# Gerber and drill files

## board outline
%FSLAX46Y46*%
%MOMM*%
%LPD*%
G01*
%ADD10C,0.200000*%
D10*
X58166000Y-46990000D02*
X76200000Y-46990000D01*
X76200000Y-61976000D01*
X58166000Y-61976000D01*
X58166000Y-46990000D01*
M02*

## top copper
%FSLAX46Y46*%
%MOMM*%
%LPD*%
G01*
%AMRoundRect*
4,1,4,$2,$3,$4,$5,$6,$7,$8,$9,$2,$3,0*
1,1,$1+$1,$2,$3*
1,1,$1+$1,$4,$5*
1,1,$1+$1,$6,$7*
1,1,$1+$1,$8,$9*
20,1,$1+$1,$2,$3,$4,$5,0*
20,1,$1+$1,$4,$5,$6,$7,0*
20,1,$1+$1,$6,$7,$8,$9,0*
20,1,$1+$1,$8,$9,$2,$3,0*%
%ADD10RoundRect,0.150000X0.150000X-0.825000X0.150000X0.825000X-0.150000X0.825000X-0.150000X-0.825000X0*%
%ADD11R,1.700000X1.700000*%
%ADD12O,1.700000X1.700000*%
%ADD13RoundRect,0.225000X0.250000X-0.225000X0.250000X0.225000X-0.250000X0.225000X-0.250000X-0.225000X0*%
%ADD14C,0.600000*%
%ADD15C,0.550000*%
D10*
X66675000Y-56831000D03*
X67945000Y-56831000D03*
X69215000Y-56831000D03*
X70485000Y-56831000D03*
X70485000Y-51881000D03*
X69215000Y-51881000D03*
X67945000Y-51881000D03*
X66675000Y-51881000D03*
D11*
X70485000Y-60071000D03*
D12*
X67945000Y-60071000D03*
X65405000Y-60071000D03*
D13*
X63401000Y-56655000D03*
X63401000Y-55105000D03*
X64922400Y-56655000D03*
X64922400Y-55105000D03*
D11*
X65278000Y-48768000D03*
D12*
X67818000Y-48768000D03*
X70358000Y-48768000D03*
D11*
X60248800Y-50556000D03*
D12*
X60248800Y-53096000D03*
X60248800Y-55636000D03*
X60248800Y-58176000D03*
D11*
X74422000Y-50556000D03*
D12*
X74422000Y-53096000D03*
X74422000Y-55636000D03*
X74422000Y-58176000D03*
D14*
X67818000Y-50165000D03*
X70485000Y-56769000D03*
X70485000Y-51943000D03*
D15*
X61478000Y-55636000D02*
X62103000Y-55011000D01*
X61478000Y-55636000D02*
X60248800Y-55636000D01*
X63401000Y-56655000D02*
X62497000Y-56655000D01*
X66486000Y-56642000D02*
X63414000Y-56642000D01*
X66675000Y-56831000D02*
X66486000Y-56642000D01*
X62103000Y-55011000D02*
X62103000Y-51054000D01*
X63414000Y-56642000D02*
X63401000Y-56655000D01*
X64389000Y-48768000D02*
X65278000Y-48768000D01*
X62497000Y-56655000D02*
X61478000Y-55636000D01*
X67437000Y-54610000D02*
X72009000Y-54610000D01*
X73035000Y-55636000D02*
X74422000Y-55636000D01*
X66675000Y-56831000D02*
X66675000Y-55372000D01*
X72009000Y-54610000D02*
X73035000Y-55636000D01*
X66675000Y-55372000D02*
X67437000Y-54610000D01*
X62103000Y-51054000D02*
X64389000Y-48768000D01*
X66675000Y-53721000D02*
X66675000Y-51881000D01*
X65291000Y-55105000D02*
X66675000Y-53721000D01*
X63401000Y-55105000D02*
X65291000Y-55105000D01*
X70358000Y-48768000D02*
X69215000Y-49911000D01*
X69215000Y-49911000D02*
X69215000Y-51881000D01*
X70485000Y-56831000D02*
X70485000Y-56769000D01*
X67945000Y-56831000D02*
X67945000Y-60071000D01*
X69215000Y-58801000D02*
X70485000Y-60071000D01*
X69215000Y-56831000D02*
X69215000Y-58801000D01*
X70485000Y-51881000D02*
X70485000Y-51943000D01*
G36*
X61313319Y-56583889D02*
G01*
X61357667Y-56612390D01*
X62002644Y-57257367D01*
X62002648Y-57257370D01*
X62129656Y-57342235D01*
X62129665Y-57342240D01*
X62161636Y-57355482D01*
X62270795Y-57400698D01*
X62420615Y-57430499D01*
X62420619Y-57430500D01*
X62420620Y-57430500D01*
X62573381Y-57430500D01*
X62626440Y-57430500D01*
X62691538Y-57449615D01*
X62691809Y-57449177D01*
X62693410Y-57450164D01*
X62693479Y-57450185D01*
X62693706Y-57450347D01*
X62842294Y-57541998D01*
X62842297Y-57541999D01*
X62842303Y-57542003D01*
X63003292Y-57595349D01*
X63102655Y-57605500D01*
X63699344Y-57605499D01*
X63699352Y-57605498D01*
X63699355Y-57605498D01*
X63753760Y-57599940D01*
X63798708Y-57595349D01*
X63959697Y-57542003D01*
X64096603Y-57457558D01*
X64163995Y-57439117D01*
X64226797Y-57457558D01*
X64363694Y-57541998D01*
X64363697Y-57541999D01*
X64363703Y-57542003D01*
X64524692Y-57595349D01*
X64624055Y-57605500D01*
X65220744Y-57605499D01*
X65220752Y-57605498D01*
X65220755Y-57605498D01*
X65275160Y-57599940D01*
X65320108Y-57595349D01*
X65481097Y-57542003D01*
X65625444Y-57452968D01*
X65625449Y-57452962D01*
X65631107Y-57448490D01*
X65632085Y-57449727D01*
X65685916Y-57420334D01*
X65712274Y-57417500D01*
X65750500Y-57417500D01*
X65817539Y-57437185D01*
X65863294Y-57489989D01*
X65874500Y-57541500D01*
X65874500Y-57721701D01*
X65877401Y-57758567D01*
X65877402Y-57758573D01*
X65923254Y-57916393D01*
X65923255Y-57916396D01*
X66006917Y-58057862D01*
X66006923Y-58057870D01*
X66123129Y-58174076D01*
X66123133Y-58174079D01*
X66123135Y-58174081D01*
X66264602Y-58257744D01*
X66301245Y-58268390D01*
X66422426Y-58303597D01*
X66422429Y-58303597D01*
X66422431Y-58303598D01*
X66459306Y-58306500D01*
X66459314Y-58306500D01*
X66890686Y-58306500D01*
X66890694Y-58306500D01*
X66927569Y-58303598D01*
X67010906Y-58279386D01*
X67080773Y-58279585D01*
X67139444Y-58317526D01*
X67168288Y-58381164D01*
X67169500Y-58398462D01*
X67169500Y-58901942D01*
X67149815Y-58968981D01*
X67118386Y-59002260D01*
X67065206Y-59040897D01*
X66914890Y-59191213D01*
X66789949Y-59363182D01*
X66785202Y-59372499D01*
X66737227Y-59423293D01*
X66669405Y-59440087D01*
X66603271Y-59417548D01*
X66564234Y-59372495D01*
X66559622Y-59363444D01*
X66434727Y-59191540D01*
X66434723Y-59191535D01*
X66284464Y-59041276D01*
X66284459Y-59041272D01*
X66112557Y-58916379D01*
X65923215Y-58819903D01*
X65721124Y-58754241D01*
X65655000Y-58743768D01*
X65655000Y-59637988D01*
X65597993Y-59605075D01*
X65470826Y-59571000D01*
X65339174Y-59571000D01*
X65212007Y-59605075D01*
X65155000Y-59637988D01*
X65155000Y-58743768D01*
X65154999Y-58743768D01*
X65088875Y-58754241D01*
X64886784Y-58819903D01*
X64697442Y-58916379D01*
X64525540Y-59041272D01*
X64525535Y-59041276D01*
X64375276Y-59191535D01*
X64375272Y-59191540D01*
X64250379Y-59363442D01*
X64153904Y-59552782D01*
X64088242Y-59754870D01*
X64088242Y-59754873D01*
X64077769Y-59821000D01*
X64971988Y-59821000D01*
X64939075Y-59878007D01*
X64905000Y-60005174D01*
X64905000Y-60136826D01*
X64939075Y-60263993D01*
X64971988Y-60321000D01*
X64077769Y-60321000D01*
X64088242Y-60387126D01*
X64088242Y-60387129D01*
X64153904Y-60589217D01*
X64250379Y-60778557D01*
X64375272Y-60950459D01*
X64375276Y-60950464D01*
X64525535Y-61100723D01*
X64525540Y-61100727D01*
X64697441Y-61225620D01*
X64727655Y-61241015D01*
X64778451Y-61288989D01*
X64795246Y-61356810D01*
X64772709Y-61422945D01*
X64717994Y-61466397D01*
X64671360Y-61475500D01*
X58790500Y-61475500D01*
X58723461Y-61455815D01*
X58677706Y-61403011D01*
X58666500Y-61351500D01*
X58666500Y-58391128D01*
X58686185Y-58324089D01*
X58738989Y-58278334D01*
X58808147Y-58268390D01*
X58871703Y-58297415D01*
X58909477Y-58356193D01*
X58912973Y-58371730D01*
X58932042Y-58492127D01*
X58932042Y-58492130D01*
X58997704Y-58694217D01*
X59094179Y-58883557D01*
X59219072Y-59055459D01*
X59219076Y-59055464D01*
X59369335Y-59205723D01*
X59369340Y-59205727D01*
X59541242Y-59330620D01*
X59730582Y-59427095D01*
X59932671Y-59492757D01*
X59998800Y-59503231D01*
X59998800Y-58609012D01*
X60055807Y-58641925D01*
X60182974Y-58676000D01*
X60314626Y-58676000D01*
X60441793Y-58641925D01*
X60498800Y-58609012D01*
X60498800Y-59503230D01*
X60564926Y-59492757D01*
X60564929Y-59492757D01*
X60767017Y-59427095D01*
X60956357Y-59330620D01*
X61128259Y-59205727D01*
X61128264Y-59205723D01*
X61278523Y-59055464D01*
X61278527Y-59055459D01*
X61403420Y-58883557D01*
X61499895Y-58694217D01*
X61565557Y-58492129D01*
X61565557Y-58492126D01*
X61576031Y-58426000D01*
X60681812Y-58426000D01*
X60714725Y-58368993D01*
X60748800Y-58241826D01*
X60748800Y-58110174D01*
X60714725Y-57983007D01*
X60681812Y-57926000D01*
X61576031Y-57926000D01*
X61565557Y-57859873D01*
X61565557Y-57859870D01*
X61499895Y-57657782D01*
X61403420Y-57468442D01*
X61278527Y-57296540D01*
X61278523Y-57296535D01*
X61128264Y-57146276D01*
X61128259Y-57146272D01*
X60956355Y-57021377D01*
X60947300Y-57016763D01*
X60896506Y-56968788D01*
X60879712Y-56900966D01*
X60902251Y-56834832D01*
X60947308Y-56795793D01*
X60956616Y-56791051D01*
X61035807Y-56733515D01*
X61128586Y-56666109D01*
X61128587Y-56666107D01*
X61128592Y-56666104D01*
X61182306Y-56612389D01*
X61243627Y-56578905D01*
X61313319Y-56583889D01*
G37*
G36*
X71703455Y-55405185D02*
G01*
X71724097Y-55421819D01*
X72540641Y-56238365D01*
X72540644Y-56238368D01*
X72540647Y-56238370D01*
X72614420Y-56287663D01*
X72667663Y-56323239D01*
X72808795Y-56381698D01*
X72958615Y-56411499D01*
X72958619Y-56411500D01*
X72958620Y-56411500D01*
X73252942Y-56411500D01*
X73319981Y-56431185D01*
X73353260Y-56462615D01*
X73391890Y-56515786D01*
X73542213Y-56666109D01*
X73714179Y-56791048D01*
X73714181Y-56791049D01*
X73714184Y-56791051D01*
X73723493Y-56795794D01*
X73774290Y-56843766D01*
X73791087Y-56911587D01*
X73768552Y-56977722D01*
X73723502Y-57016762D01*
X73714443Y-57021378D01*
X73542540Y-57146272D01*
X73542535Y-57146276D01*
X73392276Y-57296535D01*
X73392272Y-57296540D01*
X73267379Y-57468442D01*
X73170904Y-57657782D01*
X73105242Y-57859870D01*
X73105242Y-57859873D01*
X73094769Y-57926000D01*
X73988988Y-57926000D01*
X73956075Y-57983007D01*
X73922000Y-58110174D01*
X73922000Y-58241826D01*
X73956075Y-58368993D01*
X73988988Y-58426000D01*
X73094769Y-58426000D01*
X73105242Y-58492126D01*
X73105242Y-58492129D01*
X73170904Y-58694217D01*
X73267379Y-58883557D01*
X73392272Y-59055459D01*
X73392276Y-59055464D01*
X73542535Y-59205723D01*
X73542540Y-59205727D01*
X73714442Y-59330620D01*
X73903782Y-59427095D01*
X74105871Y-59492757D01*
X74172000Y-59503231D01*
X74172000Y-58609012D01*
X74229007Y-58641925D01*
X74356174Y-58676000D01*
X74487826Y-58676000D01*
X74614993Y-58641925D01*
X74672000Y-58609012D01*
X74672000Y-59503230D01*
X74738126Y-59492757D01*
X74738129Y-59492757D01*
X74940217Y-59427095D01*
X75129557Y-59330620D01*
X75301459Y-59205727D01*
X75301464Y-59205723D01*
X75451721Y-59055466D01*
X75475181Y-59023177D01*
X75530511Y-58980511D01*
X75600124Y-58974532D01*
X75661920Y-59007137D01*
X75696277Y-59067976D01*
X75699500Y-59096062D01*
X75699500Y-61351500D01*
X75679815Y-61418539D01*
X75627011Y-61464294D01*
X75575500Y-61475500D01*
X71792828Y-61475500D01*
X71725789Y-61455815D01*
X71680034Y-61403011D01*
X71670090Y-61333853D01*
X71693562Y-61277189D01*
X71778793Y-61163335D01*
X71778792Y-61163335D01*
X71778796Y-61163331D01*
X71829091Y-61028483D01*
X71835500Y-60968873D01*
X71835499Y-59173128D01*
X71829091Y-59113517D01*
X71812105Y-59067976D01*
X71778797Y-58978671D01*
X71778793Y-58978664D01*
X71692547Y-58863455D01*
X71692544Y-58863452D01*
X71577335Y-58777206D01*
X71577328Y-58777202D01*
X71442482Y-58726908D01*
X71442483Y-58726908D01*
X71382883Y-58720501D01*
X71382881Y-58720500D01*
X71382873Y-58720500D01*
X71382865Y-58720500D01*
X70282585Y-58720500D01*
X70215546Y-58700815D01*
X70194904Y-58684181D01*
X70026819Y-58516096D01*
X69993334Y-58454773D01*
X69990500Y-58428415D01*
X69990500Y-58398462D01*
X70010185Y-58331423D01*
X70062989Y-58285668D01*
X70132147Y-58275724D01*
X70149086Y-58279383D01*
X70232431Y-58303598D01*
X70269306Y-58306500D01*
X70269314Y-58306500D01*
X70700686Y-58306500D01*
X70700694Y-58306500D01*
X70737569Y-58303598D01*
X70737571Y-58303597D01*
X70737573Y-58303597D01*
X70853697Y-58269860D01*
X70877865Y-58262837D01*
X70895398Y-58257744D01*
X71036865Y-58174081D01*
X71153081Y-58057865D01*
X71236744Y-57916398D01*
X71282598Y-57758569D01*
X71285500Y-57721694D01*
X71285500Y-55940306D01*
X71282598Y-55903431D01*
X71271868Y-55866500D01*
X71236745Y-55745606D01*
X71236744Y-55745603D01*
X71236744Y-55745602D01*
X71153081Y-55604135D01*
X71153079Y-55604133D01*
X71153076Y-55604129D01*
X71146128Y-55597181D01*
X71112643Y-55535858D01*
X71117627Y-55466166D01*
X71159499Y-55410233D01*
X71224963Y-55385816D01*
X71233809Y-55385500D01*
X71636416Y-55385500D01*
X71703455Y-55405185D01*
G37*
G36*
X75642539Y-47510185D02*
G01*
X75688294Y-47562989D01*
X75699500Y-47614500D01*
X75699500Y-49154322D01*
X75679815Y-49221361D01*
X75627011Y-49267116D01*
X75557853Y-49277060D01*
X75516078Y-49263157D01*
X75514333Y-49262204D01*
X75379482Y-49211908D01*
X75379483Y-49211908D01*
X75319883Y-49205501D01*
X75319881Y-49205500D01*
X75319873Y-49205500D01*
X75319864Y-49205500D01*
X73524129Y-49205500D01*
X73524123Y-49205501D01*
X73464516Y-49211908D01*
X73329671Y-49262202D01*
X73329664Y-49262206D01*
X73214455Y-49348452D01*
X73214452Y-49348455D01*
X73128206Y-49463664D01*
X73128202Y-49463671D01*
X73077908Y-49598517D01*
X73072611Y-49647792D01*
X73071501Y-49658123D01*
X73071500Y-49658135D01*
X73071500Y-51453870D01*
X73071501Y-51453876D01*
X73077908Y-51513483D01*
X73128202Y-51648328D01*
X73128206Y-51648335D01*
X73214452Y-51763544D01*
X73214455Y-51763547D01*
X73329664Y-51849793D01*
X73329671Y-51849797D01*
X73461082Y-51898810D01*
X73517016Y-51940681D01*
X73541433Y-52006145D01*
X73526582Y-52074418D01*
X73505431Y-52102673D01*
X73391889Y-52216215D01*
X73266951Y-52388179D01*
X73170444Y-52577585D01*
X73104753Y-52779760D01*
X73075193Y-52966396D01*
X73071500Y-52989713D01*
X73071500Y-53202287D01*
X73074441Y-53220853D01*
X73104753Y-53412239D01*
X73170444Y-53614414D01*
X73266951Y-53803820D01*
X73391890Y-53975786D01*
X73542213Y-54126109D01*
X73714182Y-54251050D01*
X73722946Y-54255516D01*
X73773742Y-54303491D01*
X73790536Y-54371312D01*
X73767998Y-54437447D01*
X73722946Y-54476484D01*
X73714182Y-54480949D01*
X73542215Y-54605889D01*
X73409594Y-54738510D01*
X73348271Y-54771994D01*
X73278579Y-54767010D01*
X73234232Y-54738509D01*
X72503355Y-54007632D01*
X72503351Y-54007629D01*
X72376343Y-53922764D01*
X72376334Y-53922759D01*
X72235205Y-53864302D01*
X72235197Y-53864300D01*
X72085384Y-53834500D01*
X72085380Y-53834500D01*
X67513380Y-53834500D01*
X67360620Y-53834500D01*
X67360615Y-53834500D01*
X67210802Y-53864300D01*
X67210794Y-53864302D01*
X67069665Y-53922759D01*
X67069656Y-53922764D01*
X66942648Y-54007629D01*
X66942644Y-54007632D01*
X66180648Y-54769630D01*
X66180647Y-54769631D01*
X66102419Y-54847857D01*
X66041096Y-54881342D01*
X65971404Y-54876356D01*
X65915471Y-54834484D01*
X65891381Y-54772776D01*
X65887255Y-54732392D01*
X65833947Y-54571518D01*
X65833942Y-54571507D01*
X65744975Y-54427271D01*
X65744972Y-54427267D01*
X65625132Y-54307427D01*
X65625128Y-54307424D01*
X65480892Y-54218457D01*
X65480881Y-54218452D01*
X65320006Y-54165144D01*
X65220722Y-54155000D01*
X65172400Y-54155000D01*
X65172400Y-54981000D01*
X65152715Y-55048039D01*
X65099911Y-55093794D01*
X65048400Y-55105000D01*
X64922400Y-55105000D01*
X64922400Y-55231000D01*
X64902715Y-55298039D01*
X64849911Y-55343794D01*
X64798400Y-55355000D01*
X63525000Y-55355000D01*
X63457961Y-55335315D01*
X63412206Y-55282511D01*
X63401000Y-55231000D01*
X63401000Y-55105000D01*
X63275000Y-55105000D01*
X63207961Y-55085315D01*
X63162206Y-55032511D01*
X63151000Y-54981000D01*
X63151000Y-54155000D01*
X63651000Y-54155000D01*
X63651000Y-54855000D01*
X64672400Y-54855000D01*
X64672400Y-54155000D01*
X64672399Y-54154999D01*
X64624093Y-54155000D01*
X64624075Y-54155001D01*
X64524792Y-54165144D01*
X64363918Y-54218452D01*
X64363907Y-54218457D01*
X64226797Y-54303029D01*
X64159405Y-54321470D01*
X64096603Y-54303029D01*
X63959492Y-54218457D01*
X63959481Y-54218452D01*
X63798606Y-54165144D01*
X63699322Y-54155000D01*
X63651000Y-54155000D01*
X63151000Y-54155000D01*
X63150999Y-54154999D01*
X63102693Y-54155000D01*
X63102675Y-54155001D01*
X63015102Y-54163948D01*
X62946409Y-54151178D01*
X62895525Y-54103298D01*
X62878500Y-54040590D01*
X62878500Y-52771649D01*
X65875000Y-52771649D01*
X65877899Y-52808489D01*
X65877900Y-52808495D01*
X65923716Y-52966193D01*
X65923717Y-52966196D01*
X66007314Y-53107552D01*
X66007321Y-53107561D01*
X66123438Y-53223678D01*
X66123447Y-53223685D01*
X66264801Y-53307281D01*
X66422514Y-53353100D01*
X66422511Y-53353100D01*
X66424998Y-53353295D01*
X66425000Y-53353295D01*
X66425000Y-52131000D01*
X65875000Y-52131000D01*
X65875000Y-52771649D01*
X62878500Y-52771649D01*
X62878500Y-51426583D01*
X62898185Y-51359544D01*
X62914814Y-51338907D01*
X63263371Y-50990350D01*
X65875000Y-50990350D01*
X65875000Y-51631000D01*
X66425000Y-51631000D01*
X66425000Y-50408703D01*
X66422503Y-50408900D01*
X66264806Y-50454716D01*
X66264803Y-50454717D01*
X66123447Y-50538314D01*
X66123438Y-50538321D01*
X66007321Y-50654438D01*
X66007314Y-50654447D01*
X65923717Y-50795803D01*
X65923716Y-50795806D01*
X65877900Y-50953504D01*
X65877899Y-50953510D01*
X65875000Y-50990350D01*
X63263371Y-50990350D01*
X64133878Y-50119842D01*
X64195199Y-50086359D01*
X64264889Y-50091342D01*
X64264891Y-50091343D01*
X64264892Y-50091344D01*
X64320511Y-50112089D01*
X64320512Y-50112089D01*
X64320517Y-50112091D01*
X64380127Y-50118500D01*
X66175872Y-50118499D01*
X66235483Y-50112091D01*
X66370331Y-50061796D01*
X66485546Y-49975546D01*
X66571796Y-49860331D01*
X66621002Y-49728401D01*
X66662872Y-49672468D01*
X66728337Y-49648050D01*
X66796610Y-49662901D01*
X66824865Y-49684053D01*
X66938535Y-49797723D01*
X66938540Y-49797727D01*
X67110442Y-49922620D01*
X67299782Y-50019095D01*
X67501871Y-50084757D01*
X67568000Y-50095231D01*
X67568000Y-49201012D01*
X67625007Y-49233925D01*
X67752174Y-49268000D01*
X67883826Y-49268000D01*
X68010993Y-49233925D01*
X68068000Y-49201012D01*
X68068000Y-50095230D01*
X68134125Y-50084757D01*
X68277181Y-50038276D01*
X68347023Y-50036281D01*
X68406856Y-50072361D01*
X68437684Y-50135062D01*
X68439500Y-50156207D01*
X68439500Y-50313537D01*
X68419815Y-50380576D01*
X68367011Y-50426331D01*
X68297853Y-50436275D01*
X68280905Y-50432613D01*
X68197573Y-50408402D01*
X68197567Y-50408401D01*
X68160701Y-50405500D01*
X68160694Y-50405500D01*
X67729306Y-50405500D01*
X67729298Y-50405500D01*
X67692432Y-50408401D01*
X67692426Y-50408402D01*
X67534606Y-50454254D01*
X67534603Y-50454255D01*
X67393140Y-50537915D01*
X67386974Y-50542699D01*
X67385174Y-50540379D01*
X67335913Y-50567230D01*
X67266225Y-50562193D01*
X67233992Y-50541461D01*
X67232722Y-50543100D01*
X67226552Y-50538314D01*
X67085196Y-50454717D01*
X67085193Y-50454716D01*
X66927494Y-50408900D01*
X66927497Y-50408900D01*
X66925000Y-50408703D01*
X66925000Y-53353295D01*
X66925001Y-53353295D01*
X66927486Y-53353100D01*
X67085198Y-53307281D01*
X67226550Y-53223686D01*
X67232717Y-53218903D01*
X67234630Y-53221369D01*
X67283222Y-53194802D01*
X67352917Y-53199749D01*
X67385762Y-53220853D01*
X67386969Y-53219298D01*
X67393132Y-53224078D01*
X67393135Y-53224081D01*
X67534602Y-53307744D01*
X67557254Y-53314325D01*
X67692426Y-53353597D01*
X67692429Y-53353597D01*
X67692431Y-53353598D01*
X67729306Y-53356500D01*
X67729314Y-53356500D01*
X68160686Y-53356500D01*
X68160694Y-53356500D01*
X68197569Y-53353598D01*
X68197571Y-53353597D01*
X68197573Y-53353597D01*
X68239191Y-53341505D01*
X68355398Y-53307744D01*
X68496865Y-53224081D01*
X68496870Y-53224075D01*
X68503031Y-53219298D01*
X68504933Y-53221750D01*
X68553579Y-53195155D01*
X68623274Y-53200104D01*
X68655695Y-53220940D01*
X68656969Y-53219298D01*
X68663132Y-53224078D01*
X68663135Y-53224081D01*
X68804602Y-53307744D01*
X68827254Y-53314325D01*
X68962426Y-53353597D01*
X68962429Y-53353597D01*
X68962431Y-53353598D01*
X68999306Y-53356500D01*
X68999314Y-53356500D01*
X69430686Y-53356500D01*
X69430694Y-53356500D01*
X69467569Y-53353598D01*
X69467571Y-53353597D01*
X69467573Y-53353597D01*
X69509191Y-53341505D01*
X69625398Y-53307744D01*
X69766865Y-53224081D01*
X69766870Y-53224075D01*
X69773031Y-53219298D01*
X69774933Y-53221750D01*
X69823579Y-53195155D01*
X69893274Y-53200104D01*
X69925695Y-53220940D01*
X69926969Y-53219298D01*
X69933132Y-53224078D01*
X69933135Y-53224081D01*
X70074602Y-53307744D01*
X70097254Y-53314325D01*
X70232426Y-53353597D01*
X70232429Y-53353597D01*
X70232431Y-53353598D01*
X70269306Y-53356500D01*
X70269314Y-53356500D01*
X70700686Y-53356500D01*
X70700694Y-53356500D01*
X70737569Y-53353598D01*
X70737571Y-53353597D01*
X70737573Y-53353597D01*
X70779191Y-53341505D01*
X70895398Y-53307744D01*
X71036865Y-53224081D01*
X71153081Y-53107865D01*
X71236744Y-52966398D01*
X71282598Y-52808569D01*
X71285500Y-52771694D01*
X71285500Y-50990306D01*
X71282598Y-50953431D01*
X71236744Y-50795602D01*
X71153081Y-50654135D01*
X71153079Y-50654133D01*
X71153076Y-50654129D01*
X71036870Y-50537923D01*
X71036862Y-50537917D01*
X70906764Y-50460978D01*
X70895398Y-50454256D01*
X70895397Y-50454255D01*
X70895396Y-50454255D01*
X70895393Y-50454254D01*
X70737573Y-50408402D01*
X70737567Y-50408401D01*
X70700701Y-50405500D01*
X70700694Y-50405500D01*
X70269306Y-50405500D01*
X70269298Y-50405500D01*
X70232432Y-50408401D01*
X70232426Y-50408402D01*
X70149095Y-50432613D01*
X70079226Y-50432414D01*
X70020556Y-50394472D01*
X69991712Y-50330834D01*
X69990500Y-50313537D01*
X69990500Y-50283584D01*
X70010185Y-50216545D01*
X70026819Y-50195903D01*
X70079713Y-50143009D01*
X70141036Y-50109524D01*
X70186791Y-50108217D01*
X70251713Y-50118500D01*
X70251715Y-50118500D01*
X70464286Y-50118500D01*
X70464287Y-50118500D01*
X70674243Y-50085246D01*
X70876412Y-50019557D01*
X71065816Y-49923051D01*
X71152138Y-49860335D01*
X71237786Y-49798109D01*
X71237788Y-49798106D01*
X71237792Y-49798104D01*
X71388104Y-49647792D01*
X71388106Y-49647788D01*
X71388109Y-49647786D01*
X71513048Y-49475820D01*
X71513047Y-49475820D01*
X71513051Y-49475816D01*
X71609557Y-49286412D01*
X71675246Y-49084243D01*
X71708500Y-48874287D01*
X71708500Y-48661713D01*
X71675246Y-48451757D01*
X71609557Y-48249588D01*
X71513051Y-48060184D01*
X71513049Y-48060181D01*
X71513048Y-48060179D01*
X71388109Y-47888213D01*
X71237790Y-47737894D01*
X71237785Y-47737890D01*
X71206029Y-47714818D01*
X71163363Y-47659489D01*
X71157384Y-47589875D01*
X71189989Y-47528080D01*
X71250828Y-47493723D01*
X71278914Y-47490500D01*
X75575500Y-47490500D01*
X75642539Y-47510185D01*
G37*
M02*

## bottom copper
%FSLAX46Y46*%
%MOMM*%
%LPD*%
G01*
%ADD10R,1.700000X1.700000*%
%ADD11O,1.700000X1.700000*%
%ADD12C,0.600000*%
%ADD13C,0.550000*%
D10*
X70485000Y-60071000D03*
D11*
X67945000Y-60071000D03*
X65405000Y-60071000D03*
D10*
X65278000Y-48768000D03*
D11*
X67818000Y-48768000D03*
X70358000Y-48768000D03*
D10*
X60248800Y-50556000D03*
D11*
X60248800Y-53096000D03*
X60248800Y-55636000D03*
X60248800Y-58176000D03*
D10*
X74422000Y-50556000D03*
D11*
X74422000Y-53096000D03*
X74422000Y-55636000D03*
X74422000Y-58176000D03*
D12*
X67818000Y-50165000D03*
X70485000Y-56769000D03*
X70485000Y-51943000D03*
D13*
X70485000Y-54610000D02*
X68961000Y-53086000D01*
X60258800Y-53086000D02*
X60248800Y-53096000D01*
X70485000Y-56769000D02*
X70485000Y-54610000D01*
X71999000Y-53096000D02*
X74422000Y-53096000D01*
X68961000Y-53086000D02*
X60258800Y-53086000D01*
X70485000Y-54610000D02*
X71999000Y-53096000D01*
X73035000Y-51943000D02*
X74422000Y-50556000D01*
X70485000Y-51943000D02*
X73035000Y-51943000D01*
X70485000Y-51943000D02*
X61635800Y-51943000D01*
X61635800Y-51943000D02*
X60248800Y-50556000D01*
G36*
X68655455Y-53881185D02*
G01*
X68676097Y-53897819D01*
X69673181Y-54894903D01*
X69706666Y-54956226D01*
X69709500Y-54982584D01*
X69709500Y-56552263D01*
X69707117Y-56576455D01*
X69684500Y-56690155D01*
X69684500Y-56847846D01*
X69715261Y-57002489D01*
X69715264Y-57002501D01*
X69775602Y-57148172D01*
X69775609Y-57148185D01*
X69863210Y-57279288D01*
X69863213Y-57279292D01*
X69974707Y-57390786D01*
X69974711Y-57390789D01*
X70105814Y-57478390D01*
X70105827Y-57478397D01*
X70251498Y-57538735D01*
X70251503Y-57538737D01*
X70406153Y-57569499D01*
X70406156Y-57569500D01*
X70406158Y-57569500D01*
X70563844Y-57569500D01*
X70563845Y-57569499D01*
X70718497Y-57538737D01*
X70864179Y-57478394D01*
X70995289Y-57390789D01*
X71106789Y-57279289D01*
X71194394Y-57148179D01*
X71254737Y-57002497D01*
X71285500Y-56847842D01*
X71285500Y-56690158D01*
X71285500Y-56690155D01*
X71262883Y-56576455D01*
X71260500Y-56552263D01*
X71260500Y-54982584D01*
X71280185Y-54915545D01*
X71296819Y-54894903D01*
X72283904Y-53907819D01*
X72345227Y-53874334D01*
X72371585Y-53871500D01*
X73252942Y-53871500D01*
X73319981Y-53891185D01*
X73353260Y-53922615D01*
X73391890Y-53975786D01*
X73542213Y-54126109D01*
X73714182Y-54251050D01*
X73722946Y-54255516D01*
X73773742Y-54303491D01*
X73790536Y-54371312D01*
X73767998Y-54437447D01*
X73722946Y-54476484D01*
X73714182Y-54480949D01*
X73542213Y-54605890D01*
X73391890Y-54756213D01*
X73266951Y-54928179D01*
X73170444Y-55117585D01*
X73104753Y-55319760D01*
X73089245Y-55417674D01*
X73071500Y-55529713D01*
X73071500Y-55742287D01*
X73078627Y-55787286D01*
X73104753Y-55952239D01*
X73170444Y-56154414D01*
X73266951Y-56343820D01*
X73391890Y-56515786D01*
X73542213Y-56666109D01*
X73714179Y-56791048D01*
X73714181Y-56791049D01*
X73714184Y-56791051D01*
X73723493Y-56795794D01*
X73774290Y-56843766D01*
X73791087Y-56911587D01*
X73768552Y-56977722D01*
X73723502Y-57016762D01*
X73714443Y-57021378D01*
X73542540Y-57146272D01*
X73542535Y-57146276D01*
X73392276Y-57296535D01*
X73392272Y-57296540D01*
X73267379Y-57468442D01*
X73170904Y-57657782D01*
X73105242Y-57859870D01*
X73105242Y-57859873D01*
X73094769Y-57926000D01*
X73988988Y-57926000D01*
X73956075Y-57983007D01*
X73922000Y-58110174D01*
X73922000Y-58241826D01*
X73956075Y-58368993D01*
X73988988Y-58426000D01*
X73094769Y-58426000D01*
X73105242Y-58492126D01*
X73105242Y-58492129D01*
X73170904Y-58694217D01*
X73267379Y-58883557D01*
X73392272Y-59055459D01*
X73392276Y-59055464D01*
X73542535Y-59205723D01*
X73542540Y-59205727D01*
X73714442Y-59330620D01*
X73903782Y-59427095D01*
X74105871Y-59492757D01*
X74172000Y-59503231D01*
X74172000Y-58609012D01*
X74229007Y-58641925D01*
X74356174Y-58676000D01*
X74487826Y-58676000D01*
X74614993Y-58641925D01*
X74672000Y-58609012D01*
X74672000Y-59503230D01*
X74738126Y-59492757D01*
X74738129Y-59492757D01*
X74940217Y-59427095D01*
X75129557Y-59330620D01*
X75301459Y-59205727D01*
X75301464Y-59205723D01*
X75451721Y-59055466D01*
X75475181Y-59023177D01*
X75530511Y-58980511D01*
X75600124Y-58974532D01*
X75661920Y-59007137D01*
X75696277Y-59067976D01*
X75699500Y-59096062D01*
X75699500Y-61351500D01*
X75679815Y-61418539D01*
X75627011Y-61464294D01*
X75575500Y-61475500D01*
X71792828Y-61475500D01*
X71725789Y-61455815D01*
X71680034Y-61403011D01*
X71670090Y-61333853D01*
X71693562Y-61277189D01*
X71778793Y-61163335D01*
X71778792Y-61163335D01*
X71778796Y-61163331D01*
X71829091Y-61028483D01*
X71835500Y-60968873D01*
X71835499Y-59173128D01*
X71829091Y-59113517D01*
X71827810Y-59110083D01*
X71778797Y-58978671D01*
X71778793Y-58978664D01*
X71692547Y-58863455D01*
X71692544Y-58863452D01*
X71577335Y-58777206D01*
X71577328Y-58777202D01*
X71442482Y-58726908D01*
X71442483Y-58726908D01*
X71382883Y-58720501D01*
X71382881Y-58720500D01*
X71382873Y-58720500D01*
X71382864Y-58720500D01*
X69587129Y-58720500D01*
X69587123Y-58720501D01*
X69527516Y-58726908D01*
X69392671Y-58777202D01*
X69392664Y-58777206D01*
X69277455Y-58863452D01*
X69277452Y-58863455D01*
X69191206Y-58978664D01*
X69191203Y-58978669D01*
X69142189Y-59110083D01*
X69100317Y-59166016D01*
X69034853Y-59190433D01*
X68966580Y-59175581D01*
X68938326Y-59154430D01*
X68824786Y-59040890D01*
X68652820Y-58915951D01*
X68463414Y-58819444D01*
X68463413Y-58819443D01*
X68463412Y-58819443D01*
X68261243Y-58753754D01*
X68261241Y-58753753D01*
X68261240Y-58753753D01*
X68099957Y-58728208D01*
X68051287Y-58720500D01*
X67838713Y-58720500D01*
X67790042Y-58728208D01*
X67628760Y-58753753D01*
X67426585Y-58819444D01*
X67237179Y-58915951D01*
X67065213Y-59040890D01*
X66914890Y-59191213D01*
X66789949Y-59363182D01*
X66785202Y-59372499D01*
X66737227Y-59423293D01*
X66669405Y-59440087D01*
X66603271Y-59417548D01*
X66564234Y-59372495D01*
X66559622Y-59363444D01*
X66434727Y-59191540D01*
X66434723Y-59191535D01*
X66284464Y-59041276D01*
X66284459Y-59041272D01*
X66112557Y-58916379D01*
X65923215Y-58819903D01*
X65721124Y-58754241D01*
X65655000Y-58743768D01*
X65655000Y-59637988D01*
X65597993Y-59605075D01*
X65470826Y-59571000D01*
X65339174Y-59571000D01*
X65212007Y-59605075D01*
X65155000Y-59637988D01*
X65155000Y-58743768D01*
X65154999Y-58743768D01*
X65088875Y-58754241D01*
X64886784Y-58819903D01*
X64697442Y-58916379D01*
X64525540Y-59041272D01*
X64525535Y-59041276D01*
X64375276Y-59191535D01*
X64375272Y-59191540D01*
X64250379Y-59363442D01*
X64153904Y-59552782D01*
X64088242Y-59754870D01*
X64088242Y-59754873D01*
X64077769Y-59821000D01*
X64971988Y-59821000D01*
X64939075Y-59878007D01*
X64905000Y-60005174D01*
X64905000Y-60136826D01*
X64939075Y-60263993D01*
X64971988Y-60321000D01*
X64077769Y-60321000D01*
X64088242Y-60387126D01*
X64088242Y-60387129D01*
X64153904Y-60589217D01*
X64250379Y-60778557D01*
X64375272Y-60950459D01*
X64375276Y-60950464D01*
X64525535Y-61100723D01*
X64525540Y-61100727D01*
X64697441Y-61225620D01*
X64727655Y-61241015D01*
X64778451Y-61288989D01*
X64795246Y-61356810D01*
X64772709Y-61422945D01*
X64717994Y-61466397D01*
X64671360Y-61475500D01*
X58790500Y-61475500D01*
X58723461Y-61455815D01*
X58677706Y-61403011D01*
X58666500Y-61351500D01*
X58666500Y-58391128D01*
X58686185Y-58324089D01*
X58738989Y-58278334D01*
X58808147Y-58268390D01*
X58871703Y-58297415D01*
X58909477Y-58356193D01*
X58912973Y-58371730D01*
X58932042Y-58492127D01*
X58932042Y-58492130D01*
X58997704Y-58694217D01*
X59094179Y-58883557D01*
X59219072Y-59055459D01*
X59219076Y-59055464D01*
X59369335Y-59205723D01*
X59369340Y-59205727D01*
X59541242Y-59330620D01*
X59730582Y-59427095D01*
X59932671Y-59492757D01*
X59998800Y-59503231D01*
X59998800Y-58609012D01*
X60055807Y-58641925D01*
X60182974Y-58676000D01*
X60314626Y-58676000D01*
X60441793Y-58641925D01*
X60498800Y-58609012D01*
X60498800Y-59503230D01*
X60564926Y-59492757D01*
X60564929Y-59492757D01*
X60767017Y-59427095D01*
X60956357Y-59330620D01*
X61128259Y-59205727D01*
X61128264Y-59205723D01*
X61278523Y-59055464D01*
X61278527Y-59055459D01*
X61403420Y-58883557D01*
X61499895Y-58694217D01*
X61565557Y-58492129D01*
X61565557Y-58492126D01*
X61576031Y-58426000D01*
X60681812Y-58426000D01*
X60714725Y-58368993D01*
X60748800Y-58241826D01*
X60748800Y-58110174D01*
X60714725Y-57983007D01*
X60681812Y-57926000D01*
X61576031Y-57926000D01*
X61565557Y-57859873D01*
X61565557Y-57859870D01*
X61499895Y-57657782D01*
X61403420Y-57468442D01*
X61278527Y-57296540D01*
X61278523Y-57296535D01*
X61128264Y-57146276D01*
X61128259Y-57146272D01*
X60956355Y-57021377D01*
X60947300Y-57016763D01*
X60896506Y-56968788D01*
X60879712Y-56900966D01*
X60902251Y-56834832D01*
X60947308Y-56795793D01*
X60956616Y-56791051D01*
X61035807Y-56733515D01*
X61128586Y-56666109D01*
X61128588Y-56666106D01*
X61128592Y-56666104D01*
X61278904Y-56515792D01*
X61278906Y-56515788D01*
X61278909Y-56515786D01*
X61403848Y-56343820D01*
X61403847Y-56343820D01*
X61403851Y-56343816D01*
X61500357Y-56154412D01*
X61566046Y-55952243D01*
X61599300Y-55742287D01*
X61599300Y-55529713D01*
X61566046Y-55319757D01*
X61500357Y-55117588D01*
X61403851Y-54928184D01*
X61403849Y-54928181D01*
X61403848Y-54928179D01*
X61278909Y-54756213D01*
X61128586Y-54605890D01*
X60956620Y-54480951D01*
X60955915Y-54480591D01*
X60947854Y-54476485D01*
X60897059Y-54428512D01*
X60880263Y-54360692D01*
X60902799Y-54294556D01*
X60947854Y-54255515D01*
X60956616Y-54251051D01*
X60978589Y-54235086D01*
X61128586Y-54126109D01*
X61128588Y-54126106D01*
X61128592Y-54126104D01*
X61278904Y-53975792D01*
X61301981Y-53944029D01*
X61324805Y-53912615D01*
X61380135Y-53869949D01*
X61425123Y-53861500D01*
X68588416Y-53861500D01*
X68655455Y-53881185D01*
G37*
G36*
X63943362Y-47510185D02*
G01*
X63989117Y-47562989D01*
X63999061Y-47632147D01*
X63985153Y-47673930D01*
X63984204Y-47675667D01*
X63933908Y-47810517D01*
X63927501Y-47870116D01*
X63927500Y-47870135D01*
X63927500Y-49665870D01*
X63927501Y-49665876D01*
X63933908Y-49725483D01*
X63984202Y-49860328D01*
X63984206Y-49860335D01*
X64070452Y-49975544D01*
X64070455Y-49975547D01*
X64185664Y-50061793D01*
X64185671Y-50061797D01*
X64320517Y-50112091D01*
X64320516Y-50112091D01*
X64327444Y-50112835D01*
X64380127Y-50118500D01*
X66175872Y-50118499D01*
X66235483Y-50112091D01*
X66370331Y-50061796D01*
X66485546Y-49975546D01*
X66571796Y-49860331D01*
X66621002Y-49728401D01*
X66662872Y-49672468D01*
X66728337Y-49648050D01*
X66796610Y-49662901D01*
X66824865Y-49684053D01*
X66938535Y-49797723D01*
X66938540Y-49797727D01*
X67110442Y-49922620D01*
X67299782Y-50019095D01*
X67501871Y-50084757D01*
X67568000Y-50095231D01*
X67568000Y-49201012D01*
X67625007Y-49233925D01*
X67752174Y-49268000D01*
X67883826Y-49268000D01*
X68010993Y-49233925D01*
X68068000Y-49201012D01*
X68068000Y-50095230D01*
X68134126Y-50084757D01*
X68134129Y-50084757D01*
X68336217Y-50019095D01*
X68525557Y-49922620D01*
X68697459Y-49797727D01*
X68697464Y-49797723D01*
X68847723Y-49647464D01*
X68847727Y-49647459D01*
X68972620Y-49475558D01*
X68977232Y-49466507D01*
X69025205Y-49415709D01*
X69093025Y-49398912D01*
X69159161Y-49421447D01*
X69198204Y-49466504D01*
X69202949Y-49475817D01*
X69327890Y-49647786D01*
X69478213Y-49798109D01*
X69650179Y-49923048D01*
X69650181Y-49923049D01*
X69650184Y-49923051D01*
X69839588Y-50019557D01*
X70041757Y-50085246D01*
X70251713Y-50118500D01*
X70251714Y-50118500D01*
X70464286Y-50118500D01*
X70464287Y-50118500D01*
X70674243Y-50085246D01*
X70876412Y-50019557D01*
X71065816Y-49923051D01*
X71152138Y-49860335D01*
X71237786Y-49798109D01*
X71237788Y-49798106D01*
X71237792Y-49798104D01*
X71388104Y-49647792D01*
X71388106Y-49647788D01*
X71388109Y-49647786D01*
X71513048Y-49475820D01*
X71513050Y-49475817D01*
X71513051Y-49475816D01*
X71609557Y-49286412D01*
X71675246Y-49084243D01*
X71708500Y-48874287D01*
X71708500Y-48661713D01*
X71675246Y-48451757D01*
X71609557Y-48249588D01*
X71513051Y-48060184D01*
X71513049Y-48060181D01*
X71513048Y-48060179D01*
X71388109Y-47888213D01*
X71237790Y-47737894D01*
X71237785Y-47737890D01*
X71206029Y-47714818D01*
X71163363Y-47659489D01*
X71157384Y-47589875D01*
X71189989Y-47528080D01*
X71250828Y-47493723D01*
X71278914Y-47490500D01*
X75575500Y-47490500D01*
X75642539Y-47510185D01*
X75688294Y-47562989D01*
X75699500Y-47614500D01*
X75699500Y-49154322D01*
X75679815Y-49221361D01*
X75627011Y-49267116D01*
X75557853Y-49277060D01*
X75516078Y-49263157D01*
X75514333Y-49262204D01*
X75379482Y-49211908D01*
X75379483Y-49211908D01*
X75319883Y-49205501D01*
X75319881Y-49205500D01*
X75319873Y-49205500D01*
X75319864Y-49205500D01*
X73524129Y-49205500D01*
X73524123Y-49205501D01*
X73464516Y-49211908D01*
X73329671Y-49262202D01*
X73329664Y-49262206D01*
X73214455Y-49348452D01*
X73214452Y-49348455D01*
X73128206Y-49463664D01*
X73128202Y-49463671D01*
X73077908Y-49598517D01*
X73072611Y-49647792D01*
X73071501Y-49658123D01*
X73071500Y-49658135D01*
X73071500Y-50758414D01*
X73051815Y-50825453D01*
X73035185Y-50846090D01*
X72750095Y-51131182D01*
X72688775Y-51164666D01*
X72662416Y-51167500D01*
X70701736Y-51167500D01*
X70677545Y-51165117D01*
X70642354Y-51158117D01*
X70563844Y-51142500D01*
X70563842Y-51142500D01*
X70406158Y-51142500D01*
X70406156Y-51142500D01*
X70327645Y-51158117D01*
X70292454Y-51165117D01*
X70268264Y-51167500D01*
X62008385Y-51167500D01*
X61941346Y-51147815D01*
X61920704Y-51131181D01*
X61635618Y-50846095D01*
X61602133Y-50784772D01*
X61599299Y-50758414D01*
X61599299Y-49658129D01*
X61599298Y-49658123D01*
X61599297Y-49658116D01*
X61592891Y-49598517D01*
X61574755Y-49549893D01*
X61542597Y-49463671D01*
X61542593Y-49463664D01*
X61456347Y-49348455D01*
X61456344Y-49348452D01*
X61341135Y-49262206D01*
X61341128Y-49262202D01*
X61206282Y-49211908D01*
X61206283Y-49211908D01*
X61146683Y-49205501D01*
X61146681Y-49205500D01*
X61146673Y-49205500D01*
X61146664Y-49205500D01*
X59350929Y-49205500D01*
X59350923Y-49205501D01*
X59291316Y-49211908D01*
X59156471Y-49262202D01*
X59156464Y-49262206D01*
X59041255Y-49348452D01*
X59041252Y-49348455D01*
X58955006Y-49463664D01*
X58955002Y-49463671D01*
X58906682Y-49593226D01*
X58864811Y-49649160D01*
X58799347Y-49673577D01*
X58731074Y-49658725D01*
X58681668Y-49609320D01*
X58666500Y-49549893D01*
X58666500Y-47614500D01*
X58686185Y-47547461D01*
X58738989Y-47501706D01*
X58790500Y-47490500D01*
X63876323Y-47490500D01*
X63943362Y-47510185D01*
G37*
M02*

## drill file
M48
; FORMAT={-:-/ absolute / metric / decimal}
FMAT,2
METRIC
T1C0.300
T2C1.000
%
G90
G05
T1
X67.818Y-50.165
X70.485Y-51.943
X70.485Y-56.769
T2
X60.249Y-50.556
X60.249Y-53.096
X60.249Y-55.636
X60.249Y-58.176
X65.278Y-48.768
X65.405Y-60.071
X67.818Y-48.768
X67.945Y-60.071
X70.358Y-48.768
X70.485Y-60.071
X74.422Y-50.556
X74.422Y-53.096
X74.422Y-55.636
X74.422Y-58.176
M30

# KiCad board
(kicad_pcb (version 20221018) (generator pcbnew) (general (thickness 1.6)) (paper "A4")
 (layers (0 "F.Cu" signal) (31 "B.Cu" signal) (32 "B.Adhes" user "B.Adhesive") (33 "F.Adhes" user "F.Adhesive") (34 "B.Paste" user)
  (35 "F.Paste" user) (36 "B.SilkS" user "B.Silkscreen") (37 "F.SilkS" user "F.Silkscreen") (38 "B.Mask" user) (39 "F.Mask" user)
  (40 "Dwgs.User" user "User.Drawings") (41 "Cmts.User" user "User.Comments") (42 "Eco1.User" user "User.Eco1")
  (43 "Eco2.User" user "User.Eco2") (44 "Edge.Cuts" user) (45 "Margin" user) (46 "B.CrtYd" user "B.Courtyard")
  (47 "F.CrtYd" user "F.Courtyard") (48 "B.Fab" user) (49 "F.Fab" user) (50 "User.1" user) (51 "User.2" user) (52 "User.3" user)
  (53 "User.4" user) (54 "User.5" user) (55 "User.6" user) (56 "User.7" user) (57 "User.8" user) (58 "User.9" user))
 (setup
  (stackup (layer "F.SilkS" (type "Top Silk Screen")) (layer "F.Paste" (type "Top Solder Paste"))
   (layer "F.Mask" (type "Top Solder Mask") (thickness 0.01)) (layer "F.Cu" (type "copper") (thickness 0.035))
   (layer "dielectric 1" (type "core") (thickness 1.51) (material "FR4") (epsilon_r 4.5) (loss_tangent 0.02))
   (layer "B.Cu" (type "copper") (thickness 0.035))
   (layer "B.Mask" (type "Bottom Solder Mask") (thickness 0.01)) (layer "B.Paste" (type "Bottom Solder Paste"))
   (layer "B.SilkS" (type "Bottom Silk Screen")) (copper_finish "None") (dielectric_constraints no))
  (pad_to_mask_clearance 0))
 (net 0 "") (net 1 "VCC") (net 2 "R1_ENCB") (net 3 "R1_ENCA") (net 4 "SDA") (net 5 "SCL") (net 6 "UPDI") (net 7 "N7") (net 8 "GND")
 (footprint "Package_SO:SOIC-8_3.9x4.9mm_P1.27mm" (layer "F.Cu") (at 68.58 54.356 90)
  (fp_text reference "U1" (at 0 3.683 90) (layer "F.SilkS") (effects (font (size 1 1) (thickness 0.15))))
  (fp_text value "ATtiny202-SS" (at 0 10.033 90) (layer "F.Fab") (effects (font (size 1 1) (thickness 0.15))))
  (pad "1" smd roundrect (at -2.475 -1.905 90) (size 1.95 0.6) (layers "F.Cu" "F.Paste" "F.Mask") (roundrect_rratio 0.25) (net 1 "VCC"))
  (pad "2" smd roundrect (at -2.475 -0.635 90) (size 1.95 0.6) (layers "F.Cu" "F.Paste" "F.Mask") (roundrect_rratio 0.25) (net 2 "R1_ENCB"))
  (pad "3" smd roundrect (at -2.475 0.635 90) (size 1.95 0.6) (layers "F.Cu" "F.Paste" "F.Mask") (roundrect_rratio 0.25) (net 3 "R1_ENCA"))
  (pad "4" smd roundrect (at -2.475 1.905 90) (size 1.95 0.6) (layers "F.Cu" "F.Paste" "F.Mask") (roundrect_rratio 0.25) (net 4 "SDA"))
  (pad "5" smd roundrect (at 2.475 1.905 90) (size 1.95 0.6) (layers "F.Cu" "F.Paste" "F.Mask") (roundrect_rratio 0.25) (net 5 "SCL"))
  (pad "6" smd roundrect (at 2.475 0.635 90) (size 1.95 0.6) (layers "F.Cu" "F.Paste" "F.Mask") (roundrect_rratio 0.25) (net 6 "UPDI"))
  (pad "7" smd roundrect (at 2.475 -0.635 90) (size 1.95 0.6) (layers "F.Cu" "F.Paste" "F.Mask") (roundrect_rratio 0.25) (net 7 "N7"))
  (pad "8" smd roundrect (at 2.475 -1.905 90) (size 1.95 0.6) (layers "F.Cu" "F.Paste" "F.Mask") (roundrect_rratio 0.25) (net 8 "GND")))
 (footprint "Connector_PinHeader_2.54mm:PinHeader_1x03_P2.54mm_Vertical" (layer "F.Cu") (at 70.485 60.071 -90)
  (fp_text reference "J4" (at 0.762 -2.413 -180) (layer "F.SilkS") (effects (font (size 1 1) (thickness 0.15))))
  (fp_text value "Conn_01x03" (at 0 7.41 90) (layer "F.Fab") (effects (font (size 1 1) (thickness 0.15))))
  (pad "1" thru_hole rect (at 0 0 270) (size 1.7 1.7) (drill 1) (layers "*.Cu" "*.Mask") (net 3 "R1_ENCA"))
  (pad "2" thru_hole oval (at 0 2.54 270) (size 1.7 1.7) (drill 1) (layers "*.Cu" "*.Mask") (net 2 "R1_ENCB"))
  (pad "3" thru_hole oval (at 0 5.08 270) (size 1.7 1.7) (drill 1) (layers "*.Cu" "*.Mask") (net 8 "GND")))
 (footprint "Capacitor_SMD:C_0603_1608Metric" (layer "F.Cu") (at 63.401 55.88 90)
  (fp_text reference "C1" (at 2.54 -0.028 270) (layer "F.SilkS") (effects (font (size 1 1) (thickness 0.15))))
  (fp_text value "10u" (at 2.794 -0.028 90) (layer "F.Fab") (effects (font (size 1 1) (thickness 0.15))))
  (pad "1" smd roundrect (at -0.775 0 90) (size 0.9 0.95) (layers "F.Cu" "F.Paste" "F.Mask") (roundrect_rratio 0.25) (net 1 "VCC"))
  (pad "2" smd roundrect (at 0.775 0 90) (size 0.9 0.95) (layers "F.Cu" "F.Paste" "F.Mask") (roundrect_rratio 0.25) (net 8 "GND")))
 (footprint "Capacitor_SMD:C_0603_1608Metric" (layer "F.Cu") (at 64.9224 55.88 90)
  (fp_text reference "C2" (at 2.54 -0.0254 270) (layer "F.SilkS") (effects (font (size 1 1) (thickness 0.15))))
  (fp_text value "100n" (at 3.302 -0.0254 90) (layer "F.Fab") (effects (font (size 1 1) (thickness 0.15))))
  (pad "1" smd roundrect (at -0.775 0 90) (size 0.9 0.95) (layers "F.Cu" "F.Paste" "F.Mask") (roundrect_rratio 0.25) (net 1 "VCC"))
  (pad "2" smd roundrect (at 0.775 0 90) (size 0.9 0.95) (layers "F.Cu" "F.Paste" "F.Mask") (roundrect_rratio 0.25) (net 8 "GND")))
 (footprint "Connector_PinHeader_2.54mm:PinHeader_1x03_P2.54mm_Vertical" (layer "F.Cu") (at 65.278 48.768 90)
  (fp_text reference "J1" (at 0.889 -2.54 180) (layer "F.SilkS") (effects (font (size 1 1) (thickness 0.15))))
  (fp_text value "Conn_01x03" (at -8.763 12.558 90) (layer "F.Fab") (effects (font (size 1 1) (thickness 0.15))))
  (pad "1" thru_hole rect (at 0 0 90) (size 1.7 1.7) (drill 1) (layers "*.Cu" "*.Mask") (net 1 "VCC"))
  (pad "2" thru_hole oval (at 0 2.54 90) (size 1.7 1.7) (drill 1) (layers "*.Cu" "*.Mask") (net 8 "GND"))
  (pad "3" thru_hole oval (at 0 5.08 90) (size 1.7 1.7) (drill 1) (layers "*.Cu" "*.Mask") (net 6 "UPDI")))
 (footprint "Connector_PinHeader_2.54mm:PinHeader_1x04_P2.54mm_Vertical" (layer "F.Cu") (at 60.2488 50.556)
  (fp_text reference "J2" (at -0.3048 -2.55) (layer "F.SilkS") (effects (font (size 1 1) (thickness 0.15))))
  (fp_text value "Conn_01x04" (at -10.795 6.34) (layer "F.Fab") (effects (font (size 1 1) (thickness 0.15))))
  (pad "1" thru_hole rect (at 0 0) (size 1.7 1.7) (drill 1) (layers "*.Cu" "*.Mask") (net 5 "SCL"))
  (pad "2" thru_hole oval (at 0 2.54) (size 1.7 1.7) (drill 1) (layers "*.Cu" "*.Mask") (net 4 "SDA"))
  (pad "3" thru_hole oval (at 0 5.08) (size 1.7 1.7) (drill 1) (layers "*.Cu" "*.Mask") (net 1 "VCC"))
  (pad "4" thru_hole oval (at 0 7.62) (size 1.7 1.7) (drill 1) (layers "*.Cu" "*.Mask") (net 8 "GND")))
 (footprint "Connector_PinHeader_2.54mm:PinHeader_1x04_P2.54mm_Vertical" (layer "F.Cu") (at 74.422 50.556)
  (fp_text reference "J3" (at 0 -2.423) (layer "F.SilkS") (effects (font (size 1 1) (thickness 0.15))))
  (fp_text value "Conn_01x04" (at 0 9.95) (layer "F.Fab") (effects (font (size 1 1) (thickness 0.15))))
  (pad "1" thru_hole rect (at 0 0) (size 1.7 1.7) (drill 1) (layers "*.Cu" "*.Mask") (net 5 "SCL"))
  (pad "2" thru_hole oval (at 0 2.54) (size 1.7 1.7) (drill 1) (layers "*.Cu" "*.Mask") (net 4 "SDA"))
  (pad "3" thru_hole oval (at 0 5.08) (size 1.7 1.7) (drill 1) (layers "*.Cu" "*.Mask") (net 1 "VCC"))
  (pad "4" thru_hole oval (at 0 7.62) (size 1.7 1.7) (drill 1) (layers "*.Cu" "*.Mask") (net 8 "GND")))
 (gr_rect (start 58.166 46.99) (end 76.2 61.976) (stroke (width 0.2) (type default)) (fill none) (layer "Edge.Cuts"))
 (segment (start 61.478 55.636) (end 62.103 55.011) (width 0.55) (layer "F.Cu") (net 1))
 (segment (start 61.478 55.636) (end 60.2488 55.636) (width 0.55) (layer "F.Cu") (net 1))
 (segment (start 63.401 56.655) (end 62.497 56.655) (width 0.55) (layer "F.Cu") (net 1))
 (segment (start 66.486 56.642) (end 63.414 56.642) (width 0.55) (layer "F.Cu") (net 1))
 (segment (start 66.675 56.831) (end 66.486 56.642) (width 0.55) (layer "F.Cu") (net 1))
 (segment (start 62.103 55.011) (end 62.103 51.054) (width 0.55) (layer "F.Cu") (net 1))
 (segment (start 63.414 56.642) (end 63.401 56.655) (width 0.55) (layer "F.Cu") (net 1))
 (segment (start 64.389 48.768) (end 65.278 48.768) (width 0.55) (layer "F.Cu") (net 1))
 (segment (start 62.497 56.655) (end 61.478 55.636) (width 0.55) (layer "F.Cu") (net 1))
 (segment (start 67.437 54.61) (end 72.009 54.61) (width 0.55) (layer "F.Cu") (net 1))
 (segment (start 73.035 55.636) (end 74.422 55.636) (width 0.55) (layer "F.Cu") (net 1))
 (segment (start 66.675 56.831) (end 66.675 55.372) (width 0.55) (layer "F.Cu") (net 1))
 (segment (start 72.009 54.61) (end 73.035 55.636) (width 0.55) (layer "F.Cu") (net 1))
 (segment (start 66.675 55.372) (end 67.437 54.61) (width 0.55) (layer "F.Cu") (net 1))
 (segment (start 62.103 51.054) (end 64.389 48.768) (width 0.55) (layer "F.Cu") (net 1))
 (segment (start 66.675 53.721) (end 66.675 51.881) (width 0.55) (layer "F.Cu") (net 8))
 (segment (start 65.291 55.105) (end 66.675 53.721) (width 0.55) (layer "F.Cu") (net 8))
 (segment (start 63.401 55.105) (end 65.291 55.105) (width 0.55) (layer "F.Cu") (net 8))
 (via (at 67.818 50.165) (size 0.6) (drill 0.3) (layers "F.Cu" "B.Cu") (free) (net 8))
 (segment (start 70.358 48.768) (end 69.215 49.911) (width 0.55) (layer "F.Cu") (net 6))
 (segment (start 69.215 49.911) (end 69.215 51.881) (width 0.55) (layer "F.Cu") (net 6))
 (segment (start 70.485 56.831) (end 70.485 56.769) (width 0.55) (layer "F.Cu") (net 4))
 (via (at 70.485 56.769) (size 0.6) (drill 0.3) (layers "F.Cu" "B.Cu") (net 4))
 (segment (start 70.485 54.61) (end 68.961 53.086) (width 0.55) (layer "B.Cu") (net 4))
 (segment (start 60.2588 53.086) (end 60.2488 53.096) (width 0.55) (layer "B.Cu") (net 4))
 (segment (start 70.485 56.769) (end 70.485 54.61) (width 0.55) (layer "B.Cu") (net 4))
 (segment (start 71.999 53.096) (end 74.422 53.096) (width 0.55) (layer "B.Cu") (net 4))
 (segment (start 68.961 53.086) (end 60.2588 53.086) (width 0.55) (layer "B.Cu") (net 4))
 (segment (start 70.485 54.61) (end 71.999 53.096) (width 0.55) (layer "B.Cu") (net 4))
 (segment (start 67.945 56.831) (end 67.945 60.071) (width 0.55) (layer "F.Cu") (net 2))
 (segment (start 69.215 58.801) (end 70.485 60.071) (width 0.55) (layer "F.Cu") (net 3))
 (segment (start 69.215 56.831) (end 69.215 58.801) (width 0.55) (layer "F.Cu") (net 3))
 (segment (start 70.485 51.881) (end 70.485 51.943) (width 0.55) (layer "F.Cu") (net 5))
 (via (at 70.485 51.943) (size 0.6) (drill 0.3) (layers "F.Cu" "B.Cu") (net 5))
 (segment (start 73.035 51.943) (end 74.422 50.556) (width 0.55) (layer "B.Cu") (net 5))
 (segment (start 70.485 51.943) (end 73.035 51.943) (width 0.55) (layer "B.Cu") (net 5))
 (segment (start 70.485 51.943) (end 61.6358 51.943) (width 0.55) (layer "B.Cu") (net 5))
 (segment (start 61.6358 51.943) (end 60.2488 50.556) (width 0.55) (layer "B.Cu") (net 5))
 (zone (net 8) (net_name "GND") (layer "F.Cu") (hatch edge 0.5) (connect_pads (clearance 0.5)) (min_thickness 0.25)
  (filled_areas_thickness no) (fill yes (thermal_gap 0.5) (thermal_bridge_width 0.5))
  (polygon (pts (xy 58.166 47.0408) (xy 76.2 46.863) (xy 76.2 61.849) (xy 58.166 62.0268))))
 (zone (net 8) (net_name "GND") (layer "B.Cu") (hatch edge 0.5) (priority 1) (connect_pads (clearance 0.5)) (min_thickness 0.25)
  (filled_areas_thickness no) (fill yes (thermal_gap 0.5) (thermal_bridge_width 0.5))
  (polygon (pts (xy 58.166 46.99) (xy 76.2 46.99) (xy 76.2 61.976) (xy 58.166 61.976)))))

